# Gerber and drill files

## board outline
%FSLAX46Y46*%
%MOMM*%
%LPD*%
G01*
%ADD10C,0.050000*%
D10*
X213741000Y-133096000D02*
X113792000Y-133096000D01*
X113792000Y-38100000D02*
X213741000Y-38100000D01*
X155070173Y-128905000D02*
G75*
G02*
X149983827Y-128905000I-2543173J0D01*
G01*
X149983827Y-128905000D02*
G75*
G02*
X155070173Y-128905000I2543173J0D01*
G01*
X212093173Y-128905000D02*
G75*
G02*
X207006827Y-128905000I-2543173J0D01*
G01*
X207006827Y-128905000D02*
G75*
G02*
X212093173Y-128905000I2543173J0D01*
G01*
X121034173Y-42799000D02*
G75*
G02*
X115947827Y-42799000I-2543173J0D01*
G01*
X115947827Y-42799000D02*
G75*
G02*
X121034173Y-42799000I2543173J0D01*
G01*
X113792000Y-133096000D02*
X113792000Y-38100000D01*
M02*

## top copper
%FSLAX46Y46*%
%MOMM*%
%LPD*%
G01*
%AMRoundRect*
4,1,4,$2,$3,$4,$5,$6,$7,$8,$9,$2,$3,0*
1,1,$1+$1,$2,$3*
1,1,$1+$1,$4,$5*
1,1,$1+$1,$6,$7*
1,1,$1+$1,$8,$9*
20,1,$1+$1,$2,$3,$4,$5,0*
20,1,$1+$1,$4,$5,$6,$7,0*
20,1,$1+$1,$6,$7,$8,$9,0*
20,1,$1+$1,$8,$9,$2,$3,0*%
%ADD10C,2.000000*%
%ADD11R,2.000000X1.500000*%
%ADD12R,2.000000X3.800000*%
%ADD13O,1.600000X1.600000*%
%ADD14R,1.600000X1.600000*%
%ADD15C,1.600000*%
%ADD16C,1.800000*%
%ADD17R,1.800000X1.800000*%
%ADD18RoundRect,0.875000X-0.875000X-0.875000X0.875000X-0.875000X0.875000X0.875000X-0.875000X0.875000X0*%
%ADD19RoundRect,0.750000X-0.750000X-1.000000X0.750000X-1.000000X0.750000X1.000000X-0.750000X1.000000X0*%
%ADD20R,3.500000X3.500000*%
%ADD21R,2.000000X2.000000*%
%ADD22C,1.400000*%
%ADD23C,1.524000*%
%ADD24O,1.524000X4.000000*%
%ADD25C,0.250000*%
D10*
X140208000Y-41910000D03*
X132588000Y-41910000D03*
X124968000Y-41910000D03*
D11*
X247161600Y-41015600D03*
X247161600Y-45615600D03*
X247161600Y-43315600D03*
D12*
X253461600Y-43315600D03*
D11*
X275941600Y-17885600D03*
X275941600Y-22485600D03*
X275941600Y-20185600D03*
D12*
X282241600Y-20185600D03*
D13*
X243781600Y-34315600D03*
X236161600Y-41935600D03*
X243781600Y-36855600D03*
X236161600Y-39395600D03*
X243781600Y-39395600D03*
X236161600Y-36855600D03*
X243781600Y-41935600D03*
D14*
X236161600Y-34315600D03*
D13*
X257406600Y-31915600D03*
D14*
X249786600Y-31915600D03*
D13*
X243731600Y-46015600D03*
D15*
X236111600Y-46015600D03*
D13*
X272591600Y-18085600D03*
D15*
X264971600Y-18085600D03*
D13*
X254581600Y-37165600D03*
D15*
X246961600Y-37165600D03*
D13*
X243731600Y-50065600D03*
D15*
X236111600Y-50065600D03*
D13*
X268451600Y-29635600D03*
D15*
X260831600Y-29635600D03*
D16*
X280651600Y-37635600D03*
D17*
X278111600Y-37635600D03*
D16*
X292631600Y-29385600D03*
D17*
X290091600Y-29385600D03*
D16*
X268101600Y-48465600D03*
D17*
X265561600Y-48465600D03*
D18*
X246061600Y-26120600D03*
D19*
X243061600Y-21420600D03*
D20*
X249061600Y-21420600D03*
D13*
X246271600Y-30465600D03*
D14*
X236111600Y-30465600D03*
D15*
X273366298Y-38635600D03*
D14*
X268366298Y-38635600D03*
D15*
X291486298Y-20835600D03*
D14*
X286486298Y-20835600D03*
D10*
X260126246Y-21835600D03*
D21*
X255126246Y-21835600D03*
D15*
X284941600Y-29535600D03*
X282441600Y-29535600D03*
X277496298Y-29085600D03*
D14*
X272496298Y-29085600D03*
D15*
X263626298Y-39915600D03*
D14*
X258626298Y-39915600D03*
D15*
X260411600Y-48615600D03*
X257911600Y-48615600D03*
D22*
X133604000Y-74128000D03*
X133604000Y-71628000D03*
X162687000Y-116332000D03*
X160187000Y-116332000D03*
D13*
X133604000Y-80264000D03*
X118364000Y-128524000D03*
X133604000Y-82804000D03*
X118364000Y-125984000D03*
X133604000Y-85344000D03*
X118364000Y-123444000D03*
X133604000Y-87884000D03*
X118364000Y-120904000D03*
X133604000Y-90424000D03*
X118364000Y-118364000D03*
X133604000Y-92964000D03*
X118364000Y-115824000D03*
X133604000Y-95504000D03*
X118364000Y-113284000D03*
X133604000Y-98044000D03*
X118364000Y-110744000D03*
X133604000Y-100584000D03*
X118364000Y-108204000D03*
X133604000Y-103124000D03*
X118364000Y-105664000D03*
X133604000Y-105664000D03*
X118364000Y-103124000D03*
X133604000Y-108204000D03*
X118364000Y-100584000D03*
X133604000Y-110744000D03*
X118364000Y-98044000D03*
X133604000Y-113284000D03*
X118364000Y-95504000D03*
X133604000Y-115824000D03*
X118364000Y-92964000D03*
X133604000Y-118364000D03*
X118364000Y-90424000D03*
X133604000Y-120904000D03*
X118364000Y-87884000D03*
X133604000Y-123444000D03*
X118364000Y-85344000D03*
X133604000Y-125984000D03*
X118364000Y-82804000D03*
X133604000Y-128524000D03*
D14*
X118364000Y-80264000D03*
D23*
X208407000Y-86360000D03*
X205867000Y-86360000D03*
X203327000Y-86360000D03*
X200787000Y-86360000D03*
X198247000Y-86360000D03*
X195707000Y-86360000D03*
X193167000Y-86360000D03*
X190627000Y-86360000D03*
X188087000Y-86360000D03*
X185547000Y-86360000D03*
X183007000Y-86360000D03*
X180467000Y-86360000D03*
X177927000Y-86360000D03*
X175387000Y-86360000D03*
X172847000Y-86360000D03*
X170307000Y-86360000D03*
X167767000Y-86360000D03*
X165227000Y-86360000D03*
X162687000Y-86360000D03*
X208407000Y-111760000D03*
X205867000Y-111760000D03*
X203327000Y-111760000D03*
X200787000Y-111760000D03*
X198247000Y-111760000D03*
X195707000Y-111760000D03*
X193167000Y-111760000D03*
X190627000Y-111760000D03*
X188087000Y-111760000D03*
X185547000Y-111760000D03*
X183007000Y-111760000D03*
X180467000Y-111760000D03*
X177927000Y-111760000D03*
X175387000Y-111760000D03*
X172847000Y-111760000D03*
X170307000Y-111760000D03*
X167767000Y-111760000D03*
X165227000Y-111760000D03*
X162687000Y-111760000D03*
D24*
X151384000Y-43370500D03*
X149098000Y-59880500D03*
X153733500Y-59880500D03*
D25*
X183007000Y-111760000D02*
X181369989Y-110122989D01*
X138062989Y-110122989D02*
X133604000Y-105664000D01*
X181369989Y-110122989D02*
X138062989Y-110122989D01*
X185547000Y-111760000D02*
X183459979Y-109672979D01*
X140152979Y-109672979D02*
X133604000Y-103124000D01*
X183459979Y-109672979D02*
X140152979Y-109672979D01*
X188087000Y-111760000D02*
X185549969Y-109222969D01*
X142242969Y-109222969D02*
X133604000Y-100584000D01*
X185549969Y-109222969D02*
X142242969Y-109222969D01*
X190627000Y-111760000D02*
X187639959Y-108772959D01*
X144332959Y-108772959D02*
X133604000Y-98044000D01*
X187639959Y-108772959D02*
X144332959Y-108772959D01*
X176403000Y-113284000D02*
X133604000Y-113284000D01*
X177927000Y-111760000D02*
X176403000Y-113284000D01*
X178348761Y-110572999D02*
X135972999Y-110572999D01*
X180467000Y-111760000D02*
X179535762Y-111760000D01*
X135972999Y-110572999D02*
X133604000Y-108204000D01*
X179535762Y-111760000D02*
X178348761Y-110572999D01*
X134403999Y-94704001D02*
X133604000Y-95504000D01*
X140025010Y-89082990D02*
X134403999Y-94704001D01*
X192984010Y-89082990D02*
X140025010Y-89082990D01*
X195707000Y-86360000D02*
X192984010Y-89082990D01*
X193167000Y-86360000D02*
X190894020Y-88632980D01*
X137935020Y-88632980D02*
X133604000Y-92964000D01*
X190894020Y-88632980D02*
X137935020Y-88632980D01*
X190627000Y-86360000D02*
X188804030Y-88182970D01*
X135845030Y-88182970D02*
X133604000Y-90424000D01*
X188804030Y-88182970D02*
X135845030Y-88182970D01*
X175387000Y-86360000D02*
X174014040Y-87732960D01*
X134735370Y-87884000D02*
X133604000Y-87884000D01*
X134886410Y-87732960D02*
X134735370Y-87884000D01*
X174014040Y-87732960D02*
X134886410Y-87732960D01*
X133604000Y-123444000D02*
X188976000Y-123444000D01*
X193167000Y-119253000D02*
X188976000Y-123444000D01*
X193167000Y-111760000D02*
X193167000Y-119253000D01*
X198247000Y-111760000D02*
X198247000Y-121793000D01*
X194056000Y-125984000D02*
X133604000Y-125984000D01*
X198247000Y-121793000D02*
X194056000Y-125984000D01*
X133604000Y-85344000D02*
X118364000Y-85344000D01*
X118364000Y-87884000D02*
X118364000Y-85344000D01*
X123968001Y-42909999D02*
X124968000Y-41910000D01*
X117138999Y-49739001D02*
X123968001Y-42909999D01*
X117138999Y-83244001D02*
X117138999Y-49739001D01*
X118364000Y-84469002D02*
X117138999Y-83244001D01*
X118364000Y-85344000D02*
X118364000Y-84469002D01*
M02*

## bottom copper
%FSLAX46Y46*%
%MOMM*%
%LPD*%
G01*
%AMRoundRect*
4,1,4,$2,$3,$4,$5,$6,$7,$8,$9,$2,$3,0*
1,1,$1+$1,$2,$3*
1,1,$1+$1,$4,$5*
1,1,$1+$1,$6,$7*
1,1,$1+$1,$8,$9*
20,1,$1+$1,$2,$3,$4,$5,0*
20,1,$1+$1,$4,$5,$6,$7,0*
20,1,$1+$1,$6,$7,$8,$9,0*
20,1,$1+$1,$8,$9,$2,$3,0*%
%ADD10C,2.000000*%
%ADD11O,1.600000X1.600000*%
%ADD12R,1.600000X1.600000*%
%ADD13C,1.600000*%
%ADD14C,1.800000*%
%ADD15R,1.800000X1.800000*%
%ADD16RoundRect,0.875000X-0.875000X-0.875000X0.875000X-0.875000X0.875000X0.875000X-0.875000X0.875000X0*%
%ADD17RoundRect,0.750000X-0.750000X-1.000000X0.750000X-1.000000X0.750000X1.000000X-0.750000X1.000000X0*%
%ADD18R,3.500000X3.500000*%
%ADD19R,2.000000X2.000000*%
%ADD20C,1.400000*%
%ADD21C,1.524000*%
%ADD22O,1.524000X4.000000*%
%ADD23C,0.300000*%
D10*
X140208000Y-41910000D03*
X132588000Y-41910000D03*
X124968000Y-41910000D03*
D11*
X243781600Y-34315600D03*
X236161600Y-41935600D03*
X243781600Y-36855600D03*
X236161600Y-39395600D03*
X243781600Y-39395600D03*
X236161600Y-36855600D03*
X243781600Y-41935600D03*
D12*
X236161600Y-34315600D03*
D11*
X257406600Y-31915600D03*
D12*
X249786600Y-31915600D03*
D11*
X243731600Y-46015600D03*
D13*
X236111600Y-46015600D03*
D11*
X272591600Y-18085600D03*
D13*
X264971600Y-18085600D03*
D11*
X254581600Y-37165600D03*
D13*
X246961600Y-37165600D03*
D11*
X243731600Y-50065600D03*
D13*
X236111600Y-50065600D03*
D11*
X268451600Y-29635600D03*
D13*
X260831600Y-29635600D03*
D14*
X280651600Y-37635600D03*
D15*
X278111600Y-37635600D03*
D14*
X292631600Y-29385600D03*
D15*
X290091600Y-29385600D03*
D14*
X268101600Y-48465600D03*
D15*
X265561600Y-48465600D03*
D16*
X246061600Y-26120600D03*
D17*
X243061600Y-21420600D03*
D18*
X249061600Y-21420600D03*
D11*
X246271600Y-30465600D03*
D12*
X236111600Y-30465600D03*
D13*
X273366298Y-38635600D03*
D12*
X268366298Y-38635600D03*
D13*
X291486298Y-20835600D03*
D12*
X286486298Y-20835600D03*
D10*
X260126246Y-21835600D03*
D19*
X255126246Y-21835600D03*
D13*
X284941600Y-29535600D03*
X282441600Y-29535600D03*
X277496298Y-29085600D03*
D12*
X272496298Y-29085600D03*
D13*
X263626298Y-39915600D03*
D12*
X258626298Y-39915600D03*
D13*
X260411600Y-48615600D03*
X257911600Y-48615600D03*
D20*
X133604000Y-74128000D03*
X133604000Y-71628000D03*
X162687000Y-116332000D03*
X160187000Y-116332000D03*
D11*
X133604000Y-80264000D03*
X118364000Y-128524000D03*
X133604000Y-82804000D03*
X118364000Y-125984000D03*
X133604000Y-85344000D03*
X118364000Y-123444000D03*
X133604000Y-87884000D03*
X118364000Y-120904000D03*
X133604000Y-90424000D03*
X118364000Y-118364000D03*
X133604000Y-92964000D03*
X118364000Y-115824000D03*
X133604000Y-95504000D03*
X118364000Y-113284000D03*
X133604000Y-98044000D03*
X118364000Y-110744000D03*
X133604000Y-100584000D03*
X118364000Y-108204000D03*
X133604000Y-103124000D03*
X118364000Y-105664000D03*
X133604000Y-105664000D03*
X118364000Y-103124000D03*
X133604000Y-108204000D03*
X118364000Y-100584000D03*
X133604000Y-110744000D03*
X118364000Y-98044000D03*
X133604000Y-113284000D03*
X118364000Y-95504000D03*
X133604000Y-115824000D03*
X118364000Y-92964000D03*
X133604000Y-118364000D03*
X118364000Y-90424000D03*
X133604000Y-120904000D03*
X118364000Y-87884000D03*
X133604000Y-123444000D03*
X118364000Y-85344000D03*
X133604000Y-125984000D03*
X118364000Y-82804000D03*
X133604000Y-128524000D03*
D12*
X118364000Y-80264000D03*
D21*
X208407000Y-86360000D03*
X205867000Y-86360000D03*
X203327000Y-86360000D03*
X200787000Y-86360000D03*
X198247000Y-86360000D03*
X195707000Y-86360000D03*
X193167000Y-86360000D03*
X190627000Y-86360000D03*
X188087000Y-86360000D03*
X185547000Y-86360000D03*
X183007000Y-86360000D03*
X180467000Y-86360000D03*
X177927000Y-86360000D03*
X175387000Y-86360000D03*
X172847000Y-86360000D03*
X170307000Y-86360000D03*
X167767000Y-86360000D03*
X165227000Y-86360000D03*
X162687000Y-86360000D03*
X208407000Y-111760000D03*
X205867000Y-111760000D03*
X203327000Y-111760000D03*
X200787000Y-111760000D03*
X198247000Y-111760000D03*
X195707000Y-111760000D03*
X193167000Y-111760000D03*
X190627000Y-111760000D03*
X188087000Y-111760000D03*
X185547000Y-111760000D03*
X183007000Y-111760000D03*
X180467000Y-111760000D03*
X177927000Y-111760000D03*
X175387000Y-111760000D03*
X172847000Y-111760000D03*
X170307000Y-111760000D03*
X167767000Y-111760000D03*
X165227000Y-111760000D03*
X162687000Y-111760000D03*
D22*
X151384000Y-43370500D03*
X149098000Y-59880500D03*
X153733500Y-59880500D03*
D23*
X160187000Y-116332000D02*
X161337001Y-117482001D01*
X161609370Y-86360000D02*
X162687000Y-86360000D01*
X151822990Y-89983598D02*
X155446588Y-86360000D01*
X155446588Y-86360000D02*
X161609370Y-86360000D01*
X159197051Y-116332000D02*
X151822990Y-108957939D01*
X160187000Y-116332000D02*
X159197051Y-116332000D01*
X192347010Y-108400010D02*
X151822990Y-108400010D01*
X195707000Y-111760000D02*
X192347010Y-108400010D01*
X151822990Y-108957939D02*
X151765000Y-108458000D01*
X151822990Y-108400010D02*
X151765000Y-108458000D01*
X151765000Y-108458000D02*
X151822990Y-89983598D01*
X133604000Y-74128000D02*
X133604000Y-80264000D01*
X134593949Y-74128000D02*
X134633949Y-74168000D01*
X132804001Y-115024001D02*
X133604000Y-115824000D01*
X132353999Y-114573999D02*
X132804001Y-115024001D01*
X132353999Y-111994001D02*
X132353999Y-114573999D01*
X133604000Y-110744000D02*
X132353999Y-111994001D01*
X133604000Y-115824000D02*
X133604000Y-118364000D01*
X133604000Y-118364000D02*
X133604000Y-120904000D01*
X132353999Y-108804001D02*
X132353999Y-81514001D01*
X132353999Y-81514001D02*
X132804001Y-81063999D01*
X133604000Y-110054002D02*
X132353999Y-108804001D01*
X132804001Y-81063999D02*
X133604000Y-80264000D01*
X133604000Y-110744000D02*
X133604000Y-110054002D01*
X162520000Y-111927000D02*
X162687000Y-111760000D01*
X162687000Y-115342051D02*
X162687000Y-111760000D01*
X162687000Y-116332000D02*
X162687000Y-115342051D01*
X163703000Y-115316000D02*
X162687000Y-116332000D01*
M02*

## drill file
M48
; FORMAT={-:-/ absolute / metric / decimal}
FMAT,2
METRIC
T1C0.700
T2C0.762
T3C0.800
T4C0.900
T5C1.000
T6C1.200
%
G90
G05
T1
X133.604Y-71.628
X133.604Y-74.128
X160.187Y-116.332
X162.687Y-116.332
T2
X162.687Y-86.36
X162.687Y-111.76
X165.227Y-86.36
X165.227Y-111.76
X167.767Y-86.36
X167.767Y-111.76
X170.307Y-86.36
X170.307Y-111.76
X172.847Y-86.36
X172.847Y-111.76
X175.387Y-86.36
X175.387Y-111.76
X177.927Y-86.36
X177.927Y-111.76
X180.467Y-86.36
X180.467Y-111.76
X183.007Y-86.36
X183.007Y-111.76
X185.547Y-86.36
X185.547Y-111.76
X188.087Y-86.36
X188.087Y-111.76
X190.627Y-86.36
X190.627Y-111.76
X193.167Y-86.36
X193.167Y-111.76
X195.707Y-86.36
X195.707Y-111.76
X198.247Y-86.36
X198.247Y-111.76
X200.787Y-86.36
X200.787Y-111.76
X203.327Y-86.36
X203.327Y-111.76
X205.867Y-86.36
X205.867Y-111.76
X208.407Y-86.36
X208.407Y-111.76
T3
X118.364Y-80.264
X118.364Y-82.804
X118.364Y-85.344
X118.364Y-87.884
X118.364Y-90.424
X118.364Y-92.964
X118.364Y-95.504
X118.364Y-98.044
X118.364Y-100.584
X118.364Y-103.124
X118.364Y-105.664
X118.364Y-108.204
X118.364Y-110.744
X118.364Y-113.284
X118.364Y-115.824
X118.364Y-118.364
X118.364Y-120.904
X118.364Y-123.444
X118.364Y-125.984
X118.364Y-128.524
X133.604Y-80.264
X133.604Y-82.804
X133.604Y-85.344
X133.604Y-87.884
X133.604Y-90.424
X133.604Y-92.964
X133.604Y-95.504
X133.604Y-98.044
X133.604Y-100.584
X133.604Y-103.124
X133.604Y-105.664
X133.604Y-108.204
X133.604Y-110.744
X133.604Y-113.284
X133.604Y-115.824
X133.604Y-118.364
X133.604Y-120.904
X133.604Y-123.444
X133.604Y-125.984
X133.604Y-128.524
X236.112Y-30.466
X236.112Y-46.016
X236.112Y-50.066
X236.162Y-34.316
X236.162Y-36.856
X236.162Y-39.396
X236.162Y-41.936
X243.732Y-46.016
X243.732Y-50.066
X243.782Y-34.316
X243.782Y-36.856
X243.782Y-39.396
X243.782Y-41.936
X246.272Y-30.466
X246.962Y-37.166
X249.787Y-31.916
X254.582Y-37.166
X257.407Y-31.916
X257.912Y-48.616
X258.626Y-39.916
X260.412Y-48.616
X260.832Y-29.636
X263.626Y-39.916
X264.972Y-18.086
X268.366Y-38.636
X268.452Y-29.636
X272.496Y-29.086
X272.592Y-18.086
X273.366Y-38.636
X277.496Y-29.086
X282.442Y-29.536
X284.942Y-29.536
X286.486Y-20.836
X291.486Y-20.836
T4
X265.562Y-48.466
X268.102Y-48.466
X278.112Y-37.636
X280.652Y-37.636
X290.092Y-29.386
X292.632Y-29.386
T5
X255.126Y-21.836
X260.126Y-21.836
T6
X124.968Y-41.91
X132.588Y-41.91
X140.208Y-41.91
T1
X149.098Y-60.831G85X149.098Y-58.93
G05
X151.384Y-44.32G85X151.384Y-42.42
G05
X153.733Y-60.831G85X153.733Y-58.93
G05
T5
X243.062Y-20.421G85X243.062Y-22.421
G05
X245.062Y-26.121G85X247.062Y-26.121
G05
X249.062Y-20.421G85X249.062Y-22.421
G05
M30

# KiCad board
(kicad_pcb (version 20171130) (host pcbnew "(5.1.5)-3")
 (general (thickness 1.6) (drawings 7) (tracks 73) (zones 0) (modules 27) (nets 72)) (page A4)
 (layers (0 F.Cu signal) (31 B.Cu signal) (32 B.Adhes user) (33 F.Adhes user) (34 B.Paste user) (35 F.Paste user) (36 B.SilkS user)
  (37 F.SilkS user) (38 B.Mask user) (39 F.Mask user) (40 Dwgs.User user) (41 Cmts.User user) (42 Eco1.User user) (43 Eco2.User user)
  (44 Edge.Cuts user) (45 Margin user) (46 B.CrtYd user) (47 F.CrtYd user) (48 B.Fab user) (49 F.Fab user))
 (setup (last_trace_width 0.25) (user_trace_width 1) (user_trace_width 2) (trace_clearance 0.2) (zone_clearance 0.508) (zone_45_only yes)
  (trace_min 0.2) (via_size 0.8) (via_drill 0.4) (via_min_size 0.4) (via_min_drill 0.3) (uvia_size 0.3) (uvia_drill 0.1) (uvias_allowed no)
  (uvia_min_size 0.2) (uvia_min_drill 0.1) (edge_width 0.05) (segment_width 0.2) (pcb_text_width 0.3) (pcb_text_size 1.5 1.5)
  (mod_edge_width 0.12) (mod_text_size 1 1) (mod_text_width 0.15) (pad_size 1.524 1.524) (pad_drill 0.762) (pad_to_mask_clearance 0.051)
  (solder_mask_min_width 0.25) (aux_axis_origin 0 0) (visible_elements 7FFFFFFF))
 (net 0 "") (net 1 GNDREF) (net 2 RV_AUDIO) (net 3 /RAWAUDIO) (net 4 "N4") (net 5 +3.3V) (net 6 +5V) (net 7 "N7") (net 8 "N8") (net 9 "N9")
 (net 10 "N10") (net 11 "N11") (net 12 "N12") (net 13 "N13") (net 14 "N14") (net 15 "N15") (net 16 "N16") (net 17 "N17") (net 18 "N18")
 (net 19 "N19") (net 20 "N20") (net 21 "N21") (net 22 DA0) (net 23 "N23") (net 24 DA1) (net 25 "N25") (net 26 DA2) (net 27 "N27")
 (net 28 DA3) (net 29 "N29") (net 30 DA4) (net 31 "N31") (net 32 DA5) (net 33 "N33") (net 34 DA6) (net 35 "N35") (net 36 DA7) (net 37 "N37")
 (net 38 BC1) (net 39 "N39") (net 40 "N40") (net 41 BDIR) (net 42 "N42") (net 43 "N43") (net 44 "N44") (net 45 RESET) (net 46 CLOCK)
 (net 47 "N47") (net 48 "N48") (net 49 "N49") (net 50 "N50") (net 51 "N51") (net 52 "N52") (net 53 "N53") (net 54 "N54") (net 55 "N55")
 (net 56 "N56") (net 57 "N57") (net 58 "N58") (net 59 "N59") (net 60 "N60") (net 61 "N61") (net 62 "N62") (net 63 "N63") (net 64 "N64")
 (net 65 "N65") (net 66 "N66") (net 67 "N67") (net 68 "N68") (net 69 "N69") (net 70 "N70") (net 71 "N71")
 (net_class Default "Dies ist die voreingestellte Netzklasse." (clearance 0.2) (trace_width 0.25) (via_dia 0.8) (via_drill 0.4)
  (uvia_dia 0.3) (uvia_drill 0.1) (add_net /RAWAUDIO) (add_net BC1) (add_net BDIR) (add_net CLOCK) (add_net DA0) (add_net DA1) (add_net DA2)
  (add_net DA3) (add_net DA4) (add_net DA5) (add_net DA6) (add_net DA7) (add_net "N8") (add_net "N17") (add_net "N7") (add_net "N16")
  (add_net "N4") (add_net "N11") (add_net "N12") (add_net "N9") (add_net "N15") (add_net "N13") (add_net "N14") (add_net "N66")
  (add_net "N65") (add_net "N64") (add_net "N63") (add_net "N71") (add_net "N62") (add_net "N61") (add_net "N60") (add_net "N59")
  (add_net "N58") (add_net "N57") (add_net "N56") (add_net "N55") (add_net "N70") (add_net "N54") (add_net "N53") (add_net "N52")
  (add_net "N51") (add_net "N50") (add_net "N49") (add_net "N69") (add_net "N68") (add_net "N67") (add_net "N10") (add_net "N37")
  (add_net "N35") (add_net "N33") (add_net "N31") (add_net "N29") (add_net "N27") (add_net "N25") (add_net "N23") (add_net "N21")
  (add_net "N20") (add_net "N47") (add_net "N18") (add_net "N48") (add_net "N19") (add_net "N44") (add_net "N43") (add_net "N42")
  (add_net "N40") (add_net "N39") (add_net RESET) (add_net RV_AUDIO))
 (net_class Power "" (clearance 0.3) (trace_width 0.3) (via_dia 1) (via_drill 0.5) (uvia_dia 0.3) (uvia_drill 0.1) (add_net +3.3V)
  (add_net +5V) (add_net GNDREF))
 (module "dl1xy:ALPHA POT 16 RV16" (layer F.Cu) (at 132.588 46.863 180)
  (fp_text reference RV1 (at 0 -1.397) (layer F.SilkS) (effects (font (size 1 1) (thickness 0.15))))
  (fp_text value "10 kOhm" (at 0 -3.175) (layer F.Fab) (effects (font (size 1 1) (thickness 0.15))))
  (pad 1 thru_hole circle (at -7.62 4.953 180) (size 2 2) (drill 1.2) (layers *.Cu *.Mask) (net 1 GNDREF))
  (pad 2 thru_hole circle (at 0 4.953 180) (size 2 2) (drill 1.2) (layers *.Cu *.Mask) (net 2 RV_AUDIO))
  (pad 3 thru_hole circle (at 7.62 4.953 180) (size 2 2) (drill 1.2) (layers *.Cu *.Mask) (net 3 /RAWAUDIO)))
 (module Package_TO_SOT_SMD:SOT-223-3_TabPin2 (layer F.Cu) (at 250.3116 43.3156)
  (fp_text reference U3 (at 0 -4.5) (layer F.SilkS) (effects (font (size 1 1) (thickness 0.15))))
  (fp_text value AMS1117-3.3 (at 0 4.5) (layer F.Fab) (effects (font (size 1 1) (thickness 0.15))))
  (pad 1 smd rect (at -3.15 -2.3) (size 2 1.5) (layers F.Cu F.Paste F.Mask) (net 1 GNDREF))
  (pad 3 smd rect (at -3.15 2.3) (size 2 1.5) (layers F.Cu F.Paste F.Mask) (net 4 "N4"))
  (pad 2 smd rect (at -3.15 0) (size 2 1.5) (layers F.Cu F.Paste F.Mask) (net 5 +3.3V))
  (pad 2 smd rect (at 3.15 0) (size 2 3.8) (layers F.Cu F.Paste F.Mask) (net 5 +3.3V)))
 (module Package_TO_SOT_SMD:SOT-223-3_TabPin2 (layer F.Cu) (at 279.0916 20.1856)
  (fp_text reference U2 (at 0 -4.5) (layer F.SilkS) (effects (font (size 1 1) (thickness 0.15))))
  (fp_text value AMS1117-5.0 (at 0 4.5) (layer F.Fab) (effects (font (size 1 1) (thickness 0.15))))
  (pad 1 smd rect (at -3.15 -2.3) (size 2 1.5) (layers F.Cu F.Paste F.Mask) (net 1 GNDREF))
  (pad 3 smd rect (at -3.15 2.3) (size 2 1.5) (layers F.Cu F.Paste F.Mask) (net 4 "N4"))
  (pad 2 smd rect (at -3.15 0) (size 2 1.5) (layers F.Cu F.Paste F.Mask) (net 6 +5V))
  (pad 2 smd rect (at 3.15 0) (size 2 3.8) (layers F.Cu F.Paste F.Mask) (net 6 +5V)))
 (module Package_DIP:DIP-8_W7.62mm (layer F.Cu) (at 236.1616 34.3156)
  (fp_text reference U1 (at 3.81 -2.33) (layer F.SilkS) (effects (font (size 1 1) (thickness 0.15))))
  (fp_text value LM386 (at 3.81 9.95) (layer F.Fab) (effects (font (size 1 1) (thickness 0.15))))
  (pad 8 thru_hole oval (at 7.62 0) (size 1.6 1.6) (drill 0.8) (layers *.Cu *.Mask) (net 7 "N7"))
  (pad 4 thru_hole oval (at 0 7.62) (size 1.6 1.6) (drill 0.8) (layers *.Cu *.Mask) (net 1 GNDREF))
  (pad 7 thru_hole oval (at 7.62 2.54) (size 1.6 1.6) (drill 0.8) (layers *.Cu *.Mask) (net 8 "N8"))
  (pad 3 thru_hole oval (at 0 5.08) (size 1.6 1.6) (drill 0.8) (layers *.Cu *.Mask) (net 2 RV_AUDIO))
  (pad 6 thru_hole oval (at 7.62 5.08) (size 1.6 1.6) (drill 0.8) (layers *.Cu *.Mask) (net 6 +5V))
  (pad 2 thru_hole oval (at 0 2.54) (size 1.6 1.6) (drill 0.8) (layers *.Cu *.Mask) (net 1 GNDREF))
  (pad 5 thru_hole oval (at 7.62 7.62) (size 1.6 1.6) (drill 0.8) (layers *.Cu *.Mask) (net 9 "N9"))
  (pad 1 thru_hole rect (at 0 0) (size 1.6 1.6) (drill 0.8) (layers *.Cu *.Mask) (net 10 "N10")))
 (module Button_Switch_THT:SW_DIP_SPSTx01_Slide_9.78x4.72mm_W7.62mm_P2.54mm (layer F.Cu) (at 249.7866 31.9156)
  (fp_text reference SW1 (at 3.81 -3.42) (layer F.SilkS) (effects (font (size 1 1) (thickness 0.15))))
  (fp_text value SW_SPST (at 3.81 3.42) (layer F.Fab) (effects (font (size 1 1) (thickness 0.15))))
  (pad 2 thru_hole oval (at 7.62 0) (size 1.6 1.6) (drill 0.8) (layers *.Cu *.Mask) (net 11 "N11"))
  (pad 1 thru_hole rect (at 0 0) (size 1.6 1.6) (drill 0.8) (layers *.Cu *.Mask) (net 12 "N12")))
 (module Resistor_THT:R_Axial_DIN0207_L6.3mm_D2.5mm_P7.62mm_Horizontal (layer F.Cu) (at 236.1116 46.0156)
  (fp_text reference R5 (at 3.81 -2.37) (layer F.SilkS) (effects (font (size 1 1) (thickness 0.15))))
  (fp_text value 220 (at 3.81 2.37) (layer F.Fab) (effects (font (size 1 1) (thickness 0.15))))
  (pad 2 thru_hole oval (at 7.62 0) (size 1.6 1.6) (drill 0.8) (layers *.Cu *.Mask) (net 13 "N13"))
  (pad 1 thru_hole circle (at 0 0) (size 1.6 1.6) (drill 0.8) (layers *.Cu *.Mask) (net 5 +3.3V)))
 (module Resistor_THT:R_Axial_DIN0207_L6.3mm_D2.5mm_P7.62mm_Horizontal (layer F.Cu) (at 264.9716 18.0856)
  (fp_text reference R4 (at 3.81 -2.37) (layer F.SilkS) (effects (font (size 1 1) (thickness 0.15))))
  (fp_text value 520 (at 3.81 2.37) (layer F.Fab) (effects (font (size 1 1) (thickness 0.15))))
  (pad 2 thru_hole oval (at 7.62 0) (size 1.6 1.6) (drill 0.8) (layers *.Cu *.Mask) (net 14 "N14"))
  (pad 1 thru_hole circle (at 0 0) (size 1.6 1.6) (drill 0.8) (layers *.Cu *.Mask) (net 6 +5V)))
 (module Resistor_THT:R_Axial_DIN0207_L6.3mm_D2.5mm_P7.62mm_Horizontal (layer F.Cu) (at 246.9616 37.1656)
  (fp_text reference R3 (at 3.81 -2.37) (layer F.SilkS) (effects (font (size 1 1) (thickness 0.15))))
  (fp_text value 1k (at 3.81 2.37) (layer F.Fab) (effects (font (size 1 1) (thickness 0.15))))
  (pad 2 thru_hole oval (at 7.62 0) (size 1.6 1.6) (drill 0.8) (layers *.Cu *.Mask) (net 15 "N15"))
  (pad 1 thru_hole circle (at 0 0) (size 1.6 1.6) (drill 0.8) (layers *.Cu *.Mask) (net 11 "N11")))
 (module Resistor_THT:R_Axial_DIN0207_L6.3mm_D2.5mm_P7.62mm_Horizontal (layer F.Cu) (at 236.1116 50.0656)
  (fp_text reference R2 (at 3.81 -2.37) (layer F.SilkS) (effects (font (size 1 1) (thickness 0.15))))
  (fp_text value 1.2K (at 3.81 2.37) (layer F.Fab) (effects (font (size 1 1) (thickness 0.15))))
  (pad 2 thru_hole oval (at 7.62 0) (size 1.6 1.6) (drill 0.8) (layers *.Cu *.Mask) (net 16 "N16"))
  (pad 1 thru_hole circle (at 0 0) (size 1.6 1.6) (drill 0.8) (layers *.Cu *.Mask) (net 9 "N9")))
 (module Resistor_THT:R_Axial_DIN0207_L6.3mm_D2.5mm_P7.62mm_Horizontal (layer F.Cu) (at 260.8316 29.6356)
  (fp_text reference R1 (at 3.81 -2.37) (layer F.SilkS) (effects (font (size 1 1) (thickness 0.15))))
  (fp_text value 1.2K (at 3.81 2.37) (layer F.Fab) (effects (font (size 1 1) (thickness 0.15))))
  (pad 2 thru_hole oval (at 7.62 0) (size 1.6 1.6) (drill 0.8) (layers *.Cu *.Mask) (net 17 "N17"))
  (pad 1 thru_hole circle (at 0 0) (size 1.6 1.6) (drill 0.8) (layers *.Cu *.Mask) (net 10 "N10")))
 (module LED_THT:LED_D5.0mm (layer F.Cu) (at 278.1116 37.6356)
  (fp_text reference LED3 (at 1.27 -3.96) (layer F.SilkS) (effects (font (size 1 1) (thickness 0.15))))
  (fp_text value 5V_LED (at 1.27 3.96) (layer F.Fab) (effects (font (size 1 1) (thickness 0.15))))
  (pad 2 thru_hole circle (at 2.54 0) (size 1.8 1.8) (drill 0.9) (layers *.Cu *.Mask) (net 14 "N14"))
  (pad 1 thru_hole rect (at 0 0) (size 1.8 1.8) (drill 0.9) (layers *.Cu *.Mask) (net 1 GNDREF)))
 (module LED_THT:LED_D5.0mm (layer F.Cu) (at 290.0916 29.3856)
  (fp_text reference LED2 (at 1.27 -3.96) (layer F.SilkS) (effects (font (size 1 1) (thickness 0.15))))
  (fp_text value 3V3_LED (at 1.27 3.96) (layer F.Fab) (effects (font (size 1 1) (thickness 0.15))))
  (pad 2 thru_hole circle (at 2.54 0) (size 1.8 1.8) (drill 0.9) (layers *.Cu *.Mask) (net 13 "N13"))
  (pad 1 thru_hole rect (at 0 0) (size 1.8 1.8) (drill 0.9) (layers *.Cu *.Mask) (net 1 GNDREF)))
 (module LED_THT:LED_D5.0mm (layer F.Cu) (at 265.5616 48.4656)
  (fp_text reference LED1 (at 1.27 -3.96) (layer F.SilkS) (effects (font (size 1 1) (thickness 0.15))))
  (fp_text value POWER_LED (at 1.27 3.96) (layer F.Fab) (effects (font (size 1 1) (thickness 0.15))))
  (pad 2 thru_hole circle (at 2.54 0) (size 1.8 1.8) (drill 0.9) (layers *.Cu *.Mask) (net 15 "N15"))
  (pad 1 thru_hole rect (at 0 0) (size 1.8 1.8) (drill 0.9) (layers *.Cu *.Mask) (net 1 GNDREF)))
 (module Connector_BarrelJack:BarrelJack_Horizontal (layer F.Cu) (at 249.0616 21.4206)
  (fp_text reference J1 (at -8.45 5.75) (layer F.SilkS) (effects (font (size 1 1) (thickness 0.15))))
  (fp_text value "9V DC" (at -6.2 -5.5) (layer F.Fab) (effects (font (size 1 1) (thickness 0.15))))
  (pad 3 thru_hole roundrect (at -3 4.7) (size 3.5 3.5) (drill oval 3 1) (layers *.Cu *.Mask) (roundrect_rratio 0.25))
  (pad 2 thru_hole roundrect (at -6 0) (size 3 3.5) (drill oval 1 3) (layers *.Cu *.Mask) (roundrect_rratio 0.25) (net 1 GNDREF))
  (pad 1 thru_hole rect (at 0 0) (size 3.5 3.5) (drill oval 1 3) (layers *.Cu *.Mask) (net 12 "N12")))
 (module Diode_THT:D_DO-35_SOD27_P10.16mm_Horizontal (layer F.Cu) (at 236.1116 30.4656)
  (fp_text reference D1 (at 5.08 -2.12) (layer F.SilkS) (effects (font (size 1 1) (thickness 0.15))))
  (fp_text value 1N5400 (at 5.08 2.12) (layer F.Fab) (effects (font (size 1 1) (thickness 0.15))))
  (pad 2 thru_hole oval (at 10.16 0) (size 1.6 1.6) (drill 0.8) (layers *.Cu *.Mask) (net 11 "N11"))
  (pad 1 thru_hole rect (at 0 0) (size 1.6 1.6) (drill 0.8) (layers *.Cu *.Mask) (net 4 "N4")))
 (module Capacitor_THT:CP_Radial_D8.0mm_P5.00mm (layer F.Cu) (at 268.366298 38.6356)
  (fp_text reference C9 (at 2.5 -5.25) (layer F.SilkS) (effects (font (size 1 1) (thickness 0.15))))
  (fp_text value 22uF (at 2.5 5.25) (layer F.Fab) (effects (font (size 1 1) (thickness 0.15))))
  (pad 2 thru_hole circle (at 5 0) (size 1.6 1.6) (drill 0.8) (layers *.Cu *.Mask) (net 1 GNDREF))
  (pad 1 thru_hole rect (at 0 0) (size 1.6 1.6) (drill 0.8) (layers *.Cu *.Mask) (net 5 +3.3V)))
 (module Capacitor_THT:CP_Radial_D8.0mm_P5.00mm (layer F.Cu) (at 286.486298 20.8356)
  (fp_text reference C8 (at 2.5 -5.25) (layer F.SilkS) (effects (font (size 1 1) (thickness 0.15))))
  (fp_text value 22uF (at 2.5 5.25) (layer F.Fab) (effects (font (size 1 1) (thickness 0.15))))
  (pad 2 thru_hole circle (at 5 0) (size 1.6 1.6) (drill 0.8) (layers *.Cu *.Mask) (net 1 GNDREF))
  (pad 1 thru_hole rect (at 0 0) (size 1.6 1.6) (drill 0.8) (layers *.Cu *.Mask) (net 6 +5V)))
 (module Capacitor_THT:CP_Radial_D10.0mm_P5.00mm (layer F.Cu) (at 255.126246 21.8356)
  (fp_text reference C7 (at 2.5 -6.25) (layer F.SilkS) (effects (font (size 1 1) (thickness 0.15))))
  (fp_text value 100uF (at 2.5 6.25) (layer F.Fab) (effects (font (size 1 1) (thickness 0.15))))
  (pad 2 thru_hole circle (at 5 0) (size 2 2) (drill 1) (layers *.Cu *.Mask) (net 1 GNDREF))
  (pad 1 thru_hole rect (at 0 0) (size 2 2) (drill 1) (layers *.Cu *.Mask) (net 4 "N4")))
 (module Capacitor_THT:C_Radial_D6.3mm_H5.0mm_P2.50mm (layer F.Cu) (at 282.4416 29.5356)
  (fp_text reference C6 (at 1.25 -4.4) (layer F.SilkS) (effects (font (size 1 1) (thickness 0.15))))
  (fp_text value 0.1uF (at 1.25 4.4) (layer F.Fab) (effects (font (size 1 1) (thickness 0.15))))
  (pad 2 thru_hole circle (at 2.5 0) (size 1.6 1.6) (drill 0.8) (layers *.Cu *.Mask) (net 1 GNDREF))
  (pad 1 thru_hole circle (at 0 0) (size 1.6 1.6) (drill 0.8) (layers *.Cu *.Mask) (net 16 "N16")))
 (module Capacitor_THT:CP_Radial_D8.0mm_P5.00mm (layer F.Cu) (at 272.496298 29.0856)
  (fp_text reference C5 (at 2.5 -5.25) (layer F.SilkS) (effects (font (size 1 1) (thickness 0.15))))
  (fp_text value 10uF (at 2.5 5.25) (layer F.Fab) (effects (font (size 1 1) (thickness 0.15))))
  (pad 2 thru_hole circle (at 5 0) (size 1.6 1.6) (drill 0.8) (layers *.Cu *.Mask) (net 7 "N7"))
  (pad 1 thru_hole rect (at 0 0) (size 1.6 1.6) (drill 0.8) (layers *.Cu *.Mask) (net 17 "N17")))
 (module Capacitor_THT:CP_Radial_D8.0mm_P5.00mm (layer F.Cu) (at 258.626298 39.9156)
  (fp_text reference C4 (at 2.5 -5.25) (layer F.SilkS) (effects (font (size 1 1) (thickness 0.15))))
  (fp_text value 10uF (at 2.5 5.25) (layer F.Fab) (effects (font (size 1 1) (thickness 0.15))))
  (pad 2 thru_hole circle (at 5 0) (size 1.6 1.6) (drill 0.8) (layers *.Cu *.Mask) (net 1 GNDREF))
  (pad 1 thru_hole rect (at 0 0) (size 1.6 1.6) (drill 0.8) (layers *.Cu *.Mask) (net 8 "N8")))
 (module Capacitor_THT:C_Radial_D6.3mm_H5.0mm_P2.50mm (layer F.Cu) (at 257.9116 48.6156)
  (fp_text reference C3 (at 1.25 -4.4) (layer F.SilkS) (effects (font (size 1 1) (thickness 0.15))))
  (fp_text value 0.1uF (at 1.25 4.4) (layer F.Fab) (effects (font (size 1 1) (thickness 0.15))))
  (pad 2 thru_hole circle (at 2.5 0) (size 1.6 1.6) (drill 0.8) (layers *.Cu *.Mask) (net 6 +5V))
  (pad 1 thru_hole circle (at 0 0) (size 1.6 1.6) (drill 0.8) (layers *.Cu *.Mask) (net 1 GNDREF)))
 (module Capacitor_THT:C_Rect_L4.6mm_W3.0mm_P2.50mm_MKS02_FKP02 (layer F.Cu) (at 133.604 71.628 270)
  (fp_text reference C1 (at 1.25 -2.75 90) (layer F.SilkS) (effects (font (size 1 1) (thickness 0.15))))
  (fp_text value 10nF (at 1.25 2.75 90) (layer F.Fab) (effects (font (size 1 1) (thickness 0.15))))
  (pad 2 thru_hole circle (at 2.5 0 270) (size 1.4 1.4) (drill 0.7) (layers *.Cu *.Mask) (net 6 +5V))
  (pad 1 thru_hole circle (at 0 0 270) (size 1.4 1.4) (drill 0.7) (layers *.Cu *.Mask) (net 1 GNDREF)))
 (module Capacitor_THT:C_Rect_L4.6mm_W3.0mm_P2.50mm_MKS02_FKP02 (layer F.Cu) (at 160.187 116.332)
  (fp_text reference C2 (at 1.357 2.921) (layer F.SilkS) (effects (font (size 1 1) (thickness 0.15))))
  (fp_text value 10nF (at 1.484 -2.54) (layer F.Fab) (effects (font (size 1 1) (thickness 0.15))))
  (pad 2 thru_hole circle (at 2.5 0) (size 1.4 1.4) (drill 0.7) (layers *.Cu *.Mask) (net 5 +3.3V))
  (pad 1 thru_hole circle (at 0 0) (size 1.4 1.4) (drill 0.7) (layers *.Cu *.Mask) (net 1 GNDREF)))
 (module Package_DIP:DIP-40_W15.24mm (layer F.Cu) (at 118.364 80.264)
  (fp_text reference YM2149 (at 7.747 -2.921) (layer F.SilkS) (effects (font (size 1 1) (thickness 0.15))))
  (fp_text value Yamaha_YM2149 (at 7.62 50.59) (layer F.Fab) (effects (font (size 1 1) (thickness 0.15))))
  (pad 40 thru_hole oval (at 15.24 0) (size 1.6 1.6) (drill 0.8) (layers *.Cu *.Mask) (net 6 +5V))
  (pad 20 thru_hole oval (at 0 48.26) (size 1.6 1.6) (drill 0.8) (layers *.Cu *.Mask) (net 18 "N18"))
  (pad 39 thru_hole oval (at 15.24 2.54) (size 1.6 1.6) (drill 0.8) (layers *.Cu *.Mask) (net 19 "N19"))
  (pad 19 thru_hole oval (at 0 45.72) (size 1.6 1.6) (drill 0.8) (layers *.Cu *.Mask) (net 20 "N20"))
  (pad 38 thru_hole oval (at 15.24 5.08) (size 1.6 1.6) (drill 0.8) (layers *.Cu *.Mask) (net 3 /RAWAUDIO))
  (pad 18 thru_hole oval (at 0 43.18) (size 1.6 1.6) (drill 0.8) (layers *.Cu *.Mask) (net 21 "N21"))
  (pad 37 thru_hole oval (at 15.24 7.62) (size 1.6 1.6) (drill 0.8) (layers *.Cu *.Mask) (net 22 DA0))
  (pad 17 thru_hole oval (at 0 40.64) (size 1.6 1.6) (drill 0.8) (layers *.Cu *.Mask) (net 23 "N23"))
  (pad 36 thru_hole oval (at 15.24 10.16) (size 1.6 1.6) (drill 0.8) (layers *.Cu *.Mask) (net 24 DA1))
  (pad 16 thru_hole oval (at 0 38.1) (size 1.6 1.6) (drill 0.8) (layers *.Cu *.Mask) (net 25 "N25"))
  (pad 35 thru_hole oval (at 15.24 12.7) (size 1.6 1.6) (drill 0.8) (layers *.Cu *.Mask) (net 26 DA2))
  (pad 15 thru_hole oval (at 0 35.56) (size 1.6 1.6) (drill 0.8) (layers *.Cu *.Mask) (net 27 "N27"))
  (pad 34 thru_hole oval (at 15.24 15.24) (size 1.6 1.6) (drill 0.8) (layers *.Cu *.Mask) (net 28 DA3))
  (pad 14 thru_hole oval (at 0 33.02) (size 1.6 1.6) (drill 0.8) (layers *.Cu *.Mask) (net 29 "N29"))
  (pad 33 thru_hole oval (at 15.24 17.78) (size 1.6 1.6) (drill 0.8) (layers *.Cu *.Mask) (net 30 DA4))
  (pad 13 thru_hole oval (at 0 30.48) (size 1.6 1.6) (drill 0.8) (layers *.Cu *.Mask) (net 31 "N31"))
  (pad 32 thru_hole oval (at 15.24 20.32) (size 1.6 1.6) (drill 0.8) (layers *.Cu *.Mask) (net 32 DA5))
  (pad 12 thru_hole oval (at 0 27.94) (size 1.6 1.6) (drill 0.8) (layers *.Cu *.Mask) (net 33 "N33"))
  (pad 31 thru_hole oval (at 15.24 22.86) (size 1.6 1.6) (drill 0.8) (layers *.Cu *.Mask) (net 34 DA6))
  (pad 11 thru_hole oval (at 0 25.4) (size 1.6 1.6) (drill 0.8) (layers *.Cu *.Mask) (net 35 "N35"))
  (pad 30 thru_hole oval (at 15.24 25.4) (size 1.6 1.6) (drill 0.8) (layers *.Cu *.Mask) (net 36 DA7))
  (pad 10 thru_hole oval (at 0 22.86) (size 1.6 1.6) (drill 0.8) (layers *.Cu *.Mask) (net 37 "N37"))
  (pad 29 thru_hole oval (at 15.24 27.94) (size 1.6 1.6) (drill 0.8) (layers *.Cu *.Mask) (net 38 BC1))
  (pad 9 thru_hole oval (at 0 20.32) (size 1.6 1.6) (drill 0.8) (layers *.Cu *.Mask) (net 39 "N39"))
  (pad 28 thru_hole oval (at 15.24 30.48) (size 1.6 1.6) (drill 0.8) (layers *.Cu *.Mask) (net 6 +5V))
  (pad 8 thru_hole oval (at 0 17.78) (size 1.6 1.6) (drill 0.8) (layers *.Cu *.Mask) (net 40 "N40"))
  (pad 27 thru_hole oval (at 15.24 33.02) (size 1.6 1.6) (drill 0.8) (layers *.Cu *.Mask) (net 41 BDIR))
  (pad 7 thru_hole oval (at 0 15.24) (size 1.6 1.6) (drill 0.8) (layers *.Cu *.Mask) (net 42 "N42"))
  (pad 26 thru_hole oval (at 15.24 35.56) (size 1.6 1.6) (drill 0.8) (layers *.Cu *.Mask) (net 6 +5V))
  (pad 6 thru_hole oval (at 0 12.7) (size 1.6 1.6) (drill 0.8) (layers *.Cu *.Mask) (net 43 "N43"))
  (pad 25 thru_hole oval (at 15.24 38.1) (size 1.6 1.6) (drill 0.8) (layers *.Cu *.Mask) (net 6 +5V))
  (pad 5 thru_hole oval (at 0 10.16) (size 1.6 1.6) (drill 0.8) (layers *.Cu *.Mask) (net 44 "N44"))
  (pad 24 thru_hole oval (at 15.24 40.64) (size 1.6 1.6) (drill 0.8) (layers *.Cu *.Mask) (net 6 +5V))
  (pad 4 thru_hole oval (at 0 7.62) (size 1.6 1.6) (drill 0.8) (layers *.Cu *.Mask) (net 3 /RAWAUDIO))
  (pad 23 thru_hole oval (at 15.24 43.18) (size 1.6 1.6) (drill 0.8) (layers *.Cu *.Mask) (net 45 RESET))
  (pad 3 thru_hole oval (at 0 5.08) (size 1.6 1.6) (drill 0.8) (layers *.Cu *.Mask) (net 3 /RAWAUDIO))
  (pad 22 thru_hole oval (at 15.24 45.72) (size 1.6 1.6) (drill 0.8) (layers *.Cu *.Mask) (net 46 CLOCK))
  (pad 2 thru_hole oval (at 0 2.54) (size 1.6 1.6) (drill 0.8) (layers *.Cu *.Mask) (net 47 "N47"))
  (pad 21 thru_hole oval (at 15.24 48.26) (size 1.6 1.6) (drill 0.8) (layers *.Cu *.Mask) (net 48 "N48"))
  (pad 1 thru_hole rect (at 0 0) (size 1.6 1.6) (drill 0.8) (layers *.Cu *.Mask) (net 1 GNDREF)))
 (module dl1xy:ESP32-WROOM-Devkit (layer F.Cu) (at 154.432 99.06 90)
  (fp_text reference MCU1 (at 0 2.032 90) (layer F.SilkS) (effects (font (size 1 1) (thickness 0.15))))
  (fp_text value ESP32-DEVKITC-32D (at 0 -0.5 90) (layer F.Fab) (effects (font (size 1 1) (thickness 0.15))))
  (pad 38 thru_hole circle (at 12.7 53.975 270) (size 1.524 1.524) (drill 0.762) (layers *.Cu *.Mask) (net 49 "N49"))
  (pad 37 thru_hole circle (at 12.7 51.435 270) (size 1.524 1.524) (drill 0.762) (layers *.Cu *.Mask) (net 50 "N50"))
  (pad 36 thru_hole circle (at 12.7 48.895 270) (size 1.524 1.524) (drill 0.762) (layers *.Cu *.Mask) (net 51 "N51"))
  (pad 35 thru_hole circle (at 12.7 46.355 270) (size 1.524 1.524) (drill 0.762) (layers *.Cu *.Mask) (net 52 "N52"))
  (pad 34 thru_hole circle (at 12.7 43.815 270) (size 1.524 1.524) (drill 0.762) (layers *.Cu *.Mask) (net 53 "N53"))
  (pad 33 thru_hole circle (at 12.7 41.275 270) (size 1.524 1.524) (drill 0.762) (layers *.Cu *.Mask) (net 28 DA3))
  (pad 32 thru_hole circle (at 12.7 38.735 270) (size 1.524 1.524) (drill 0.762) (layers *.Cu *.Mask) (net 26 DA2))
  (pad 31 thru_hole circle (at 12.7 36.195 270) (size 1.524 1.524) (drill 0.762) (layers *.Cu *.Mask) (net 24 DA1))
  (pad 30 thru_hole circle (at 12.7 33.655 270) (size 1.524 1.524) (drill 0.762) (layers *.Cu *.Mask) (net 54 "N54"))
  (pad 29 thru_hole circle (at 12.7 31.115 270) (size 1.524 1.524) (drill 0.762) (layers *.Cu *.Mask) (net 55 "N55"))
  (pad 28 thru_hole circle (at 12.7 28.575 270) (size 1.524 1.524) (drill 0.762) (layers *.Cu *.Mask) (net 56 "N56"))
  (pad 27 thru_hole circle (at 12.7 26.035 270) (size 1.524 1.524) (drill 0.762) (layers *.Cu *.Mask) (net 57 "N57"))
  (pad 26 thru_hole circle (at 12.7 23.495 270) (size 1.524 1.524) (drill 0.762) (layers *.Cu *.Mask) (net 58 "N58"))
  (pad 25 thru_hole circle (at 12.7 20.955 270) (size 1.524 1.524) (drill 0.762) (layers *.Cu *.Mask) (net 22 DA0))
  (pad 24 thru_hole circle (at 12.7 18.415 270) (size 1.524 1.524) (drill 0.762) (layers *.Cu *.Mask) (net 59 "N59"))
  (pad 23 thru_hole circle (at 12.7 15.875 270) (size 1.524 1.524) (drill 0.762) (layers *.Cu *.Mask) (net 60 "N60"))
  (pad 22 thru_hole circle (at 12.7 13.335 270) (size 1.524 1.524) (drill 0.762) (layers *.Cu *.Mask) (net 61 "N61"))
  (pad 21 thru_hole circle (at 12.7 10.795 270) (size 1.524 1.524) (drill 0.762) (layers *.Cu *.Mask) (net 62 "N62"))
  (pad 20 thru_hole circle (at 12.7 8.255 270) (size 1.524 1.524) (drill 0.762) (layers *.Cu *.Mask) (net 1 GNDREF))
  (pad 19 thru_hole circle (at -12.7 53.975 90) (size 1.524 1.524) (drill 0.762) (layers *.Cu *.Mask) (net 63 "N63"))
  (pad 18 thru_hole circle (at -12.7 51.435 90) (size 1.524 1.524) (drill 0.762) (layers *.Cu *.Mask) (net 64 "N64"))
  (pad 17 thru_hole circle (at -12.7 48.895 90) (size 1.524 1.524) (drill 0.762) (layers *.Cu *.Mask) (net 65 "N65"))
  (pad 16 thru_hole circle (at -12.7 46.355 90) (size 1.524 1.524) (drill 0.762) (layers *.Cu *.Mask) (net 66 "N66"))
  (pad 15 thru_hole circle (at -12.7 43.815 90) (size 1.524 1.524) (drill 0.762) (layers *.Cu *.Mask) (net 46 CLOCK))
  (pad 14 thru_hole circle (at -12.7 41.275 90) (size 1.524 1.524) (drill 0.762) (layers *.Cu *.Mask) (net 1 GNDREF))
  (pad 13 thru_hole circle (at -12.7 38.735 90) (size 1.524 1.524) (drill 0.762) (layers *.Cu *.Mask) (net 45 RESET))
  (pad 12 thru_hole circle (at -12.7 36.195 90) (size 1.524 1.524) (drill 0.762) (layers *.Cu *.Mask) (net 30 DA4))
  (pad 11 thru_hole circle (at -12.7 33.655 90) (size 1.524 1.524) (drill 0.762) (layers *.Cu *.Mask) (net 32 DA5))
  (pad 10 thru_hole circle (at -12.7 31.115 90) (size 1.524 1.524) (drill 0.762) (layers *.Cu *.Mask) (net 34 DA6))
  (pad 9 thru_hole circle (at -12.7 28.575 90) (size 1.524 1.524) (drill 0.762) (layers *.Cu *.Mask) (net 36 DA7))
  (pad 8 thru_hole circle (at -12.7 26.035 90) (size 1.524 1.524) (drill 0.762) (layers *.Cu *.Mask) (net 38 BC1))
  (pad 7 thru_hole circle (at -12.7 23.495 90) (size 1.524 1.524) (drill 0.762) (layers *.Cu *.Mask) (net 41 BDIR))
  (pad 6 thru_hole circle (at -12.7 20.955 90) (size 1.524 1.524) (drill 0.762) (layers *.Cu *.Mask) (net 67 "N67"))
  (pad 5 thru_hole circle (at -12.7 18.415 90) (size 1.524 1.524) (drill 0.762) (layers *.Cu *.Mask) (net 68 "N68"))
  (pad 4 thru_hole circle (at -12.7 15.875 90) (size 1.524 1.524) (drill 0.762) (layers *.Cu *.Mask) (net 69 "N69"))
  (pad 3 thru_hole circle (at -12.7 13.335 90) (size 1.524 1.524) (drill 0.762) (layers *.Cu *.Mask) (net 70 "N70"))
  (pad 2 thru_hole circle (at -12.7 10.795 90) (size 1.524 1.524) (drill 0.762) (layers *.Cu *.Mask) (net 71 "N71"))
  (pad 1 thru_hole circle (at -12.7 8.255 90) (size 1.524 1.524) (drill 0.762) (layers *.Cu *.Mask) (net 5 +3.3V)))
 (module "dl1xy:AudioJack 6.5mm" (layer F.Cu) (at 151.384 66.548 180)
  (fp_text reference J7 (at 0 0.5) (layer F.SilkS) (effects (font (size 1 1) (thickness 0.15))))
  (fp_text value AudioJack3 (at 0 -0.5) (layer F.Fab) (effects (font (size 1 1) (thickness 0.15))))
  (pad S thru_hole oval (at 0 23.1775 180) (size 1.524 4) (drill oval 0.7 2.6) (layers *.Cu *.Mask) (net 1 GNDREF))
  (pad T thru_hole oval (at 2.286 6.6675 180) (size 1.524 4) (drill oval 0.7 2.6) (layers *.Cu *.Mask) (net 9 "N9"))
  (pad R thru_hole oval (at -2.3495 6.6675 180) (size 1.524 4) (drill oval 0.7 2.6) (layers *.Cu *.Mask) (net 9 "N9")))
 (gr_line (start 213.741 133.096) (end 113.792 133.096) (layer Edge.Cuts) (width 0.05))
 (gr_line (start 113.792 38.1) (end 213.741 38.1) (layer Edge.Cuts) (width 0.05))
 (gr_circle (center 152.527 128.905) (end 155.067 128.778) (layer Edge.Cuts) (width 0.05))
 (gr_circle (center 209.55 128.905) (end 212.09 128.778) (layer Edge.Cuts) (width 0.05))
 (gr_circle (center 118.491 42.799) (end 121.031 42.672) (layer Edge.Cuts) (width 0.05))
 (gr_line (start 113.792 133.096) (end 113.792 38.1) (layer Edge.Cuts) (width 0.05))
 (segment (start 160.187 116.332) (end 161.337001 117.482001) (width 0.3) (layer B.Cu) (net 1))
 (segment (start 161.60937 86.36) (end 162.687 86.36) (width 0.3) (layer B.Cu) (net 1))
 (segment (start 151.82299 89.983598) (end 155.446588 86.36) (width 0.3) (layer B.Cu) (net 1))
 (segment (start 155.446588 86.36) (end 161.60937 86.36) (width 0.3) (layer B.Cu) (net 1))
 (segment (start 159.197051 116.332) (end 151.82299 108.957939) (width 0.3) (layer B.Cu) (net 1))
 (segment (start 160.187 116.332) (end 159.197051 116.332) (width 0.3) (layer B.Cu) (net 1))
 (segment (start 192.34701 108.40001) (end 151.82299 108.40001) (width 0.3) (layer B.Cu) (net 1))
 (segment (start 195.707 111.76) (end 192.34701 108.40001) (width 0.3) (layer B.Cu) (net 1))
 (segment (start 151.82299 108.957939) (end 151.765 108.458) (width 0.3) (layer B.Cu) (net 1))
 (segment (start 151.82299 108.40001) (end 151.765 108.458) (width 0.3) (layer B.Cu) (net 1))
 (segment (start 151.765 108.458) (end 151.82299 89.983598) (width 0.3) (layer B.Cu) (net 1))
 (segment (start 133.604 74.128) (end 133.604 80.264) (width 0.3) (layer B.Cu) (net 6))
 (segment (start 134.593949 74.128) (end 134.633949 74.168) (width 0.3) (layer B.Cu) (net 6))
 (segment (start 132.804001 115.024001) (end 133.604 115.824) (width 0.3) (layer B.Cu) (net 6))
 (segment (start 132.353999 114.573999) (end 132.804001 115.024001) (width 0.3) (layer B.Cu) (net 6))
 (segment (start 132.353999 111.994001) (end 132.353999 114.573999) (width 0.3) (layer B.Cu) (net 6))
 (segment (start 133.604 110.744) (end 132.353999 111.994001) (width 0.3) (layer B.Cu) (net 6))
 (segment (start 133.604 115.824) (end 133.604 118.364) (width 0.3) (layer B.Cu) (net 6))
 (segment (start 133.604 118.364) (end 133.604 120.904) (width 0.3) (layer B.Cu) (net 6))
 (segment (start 132.353999 108.804001) (end 132.353999 81.514001) (width 0.3) (layer B.Cu) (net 6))
 (segment (start 132.353999 81.514001) (end 132.804001 81.063999) (width 0.3) (layer B.Cu) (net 6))
 (segment (start 133.604 110.054002) (end 132.353999 108.804001) (width 0.3) (layer B.Cu) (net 6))
 (segment (start 132.804001 81.063999) (end 133.604 80.264) (width 0.3) (layer B.Cu) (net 6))
 (segment (start 133.604 110.744) (end 133.604 110.054002) (width 0.3) (layer B.Cu) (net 6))
 (segment (start 183.007 111.76) (end 181.369989 110.122989) (width 0.25) (layer F.Cu) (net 36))
 (segment (start 138.062989 110.122989) (end 133.604 105.664) (width 0.25) (layer F.Cu) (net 36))
 (segment (start 181.369989 110.122989) (end 138.062989 110.122989) (width 0.25) (layer F.Cu) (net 36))
 (segment (start 185.547 111.76) (end 183.459979 109.672979) (width 0.25) (layer F.Cu) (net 34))
 (segment (start 140.152979 109.672979) (end 133.604 103.124) (width 0.25) (layer F.Cu) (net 34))
 (segment (start 183.459979 109.672979) (end 140.152979 109.672979) (width 0.25) (layer F.Cu) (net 34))
 (segment (start 188.087 111.76) (end 185.549969 109.222969) (width 0.25) (layer F.Cu) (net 32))
 (segment (start 142.242969 109.222969) (end 133.604 100.584) (width 0.25) (layer F.Cu) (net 32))
 (segment (start 185.549969 109.222969) (end 142.242969 109.222969) (width 0.25) (layer F.Cu) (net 32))
 (segment (start 190.627 111.76) (end 187.639959 108.772959) (width 0.25) (layer F.Cu) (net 30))
 (segment (start 144.332959 108.772959) (end 133.604 98.044) (width 0.25) (layer F.Cu) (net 30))
 (segment (start 187.639959 108.772959) (end 144.332959 108.772959) (width 0.25) (layer F.Cu) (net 30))
 (segment (start 176.403 113.284) (end 133.604 113.284) (width 0.25) (layer F.Cu) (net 41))
 (segment (start 177.927 111.76) (end 176.403 113.284) (width 0.25) (layer F.Cu) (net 41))
 (segment (start 178.348761 110.572999) (end 135.972999 110.572999) (width 0.25) (layer F.Cu) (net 38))
 (segment (start 180.467 111.76) (end 179.535762 111.76) (width 0.25) (layer F.Cu) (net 38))
 (segment (start 135.972999 110.572999) (end 133.604 108.204) (width 0.25) (layer F.Cu) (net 38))
 (segment (start 179.535762 111.76) (end 178.348761 110.572999) (width 0.25) (layer F.Cu) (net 38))
 (segment (start 134.403999 94.704001) (end 133.604 95.504) (width 0.25) (layer F.Cu) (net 28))
 (segment (start 140.02501 89.08299) (end 134.403999 94.704001) (width 0.25) (layer F.Cu) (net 28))
 (segment (start 192.98401 89.08299) (end 140.02501 89.08299) (width 0.25) (layer F.Cu) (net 28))
 (segment (start 195.707 86.36) (end 192.98401 89.08299) (width 0.25) (layer F.Cu) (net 28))
 (segment (start 193.167 86.36) (end 190.89402 88.63298) (width 0.25) (layer F.Cu) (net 26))
 (segment (start 137.93502 88.63298) (end 133.604 92.964) (width 0.25) (layer F.Cu) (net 26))
 (segment (start 190.89402 88.63298) (end 137.93502 88.63298) (width 0.25) (layer F.Cu) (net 26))
 (segment (start 190.627 86.36) (end 188.80403 88.18297) (width 0.25) (layer F.Cu) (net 24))
 (segment (start 135.84503 88.18297) (end 133.604 90.424) (width 0.25) (layer F.Cu) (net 24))
 (segment (start 188.80403 88.18297) (end 135.84503 88.18297) (width 0.25) (layer F.Cu) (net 24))
 (segment (start 175.387 86.36) (end 174.01404 87.73296) (width 0.25) (layer F.Cu) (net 22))
 (segment (start 134.73537 87.884) (end 133.604 87.884) (width 0.25) (layer F.Cu) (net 22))
 (segment (start 134.88641 87.73296) (end 134.73537 87.884) (width 0.25) (layer F.Cu) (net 22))
 (segment (start 174.01404 87.73296) (end 134.88641 87.73296) (width 0.25) (layer F.Cu) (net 22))
 (segment (start 133.604 123.444) (end 188.976 123.444) (width 0.25) (layer F.Cu) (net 45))
 (segment (start 193.167 119.253) (end 188.976 123.444) (width 0.25) (layer F.Cu) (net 45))
 (segment (start 193.167 111.76) (end 193.167 119.253) (width 0.25) (layer F.Cu) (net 45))
 (segment (start 198.247 111.76) (end 198.247 121.793) (width 0.25) (layer F.Cu) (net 46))
 (segment (start 194.056 125.984) (end 133.604 125.984) (width 0.25) (layer F.Cu) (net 46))
 (segment (start 198.247 121.793) (end 194.056 125.984) (width 0.25) (layer F.Cu) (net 46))
 (segment (start 162.52 111.927) (end 162.687 111.76) (width 0.3) (layer B.Cu) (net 5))
 (segment (start 162.687 115.342051) (end 162.687 111.76) (width 0.3) (layer B.Cu) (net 5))
 (segment (start 162.687 116.332) (end 162.687 115.342051) (width 0.3) (layer B.Cu) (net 5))
 (segment (start 163.703 115.316) (end 162.687 116.332) (width 0.3) (layer B.Cu) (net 5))
 (segment (start 133.604 85.344) (end 118.364 85.344) (width 0.25) (layer F.Cu) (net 3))
 (segment (start 118.364 87.884) (end 118.364 85.344) (width 0.25) (layer F.Cu) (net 3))
 (segment (start 123.968001 42.909999) (end 124.968 41.91) (width 0.25) (layer F.Cu) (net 3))
 (segment (start 117.138999 49.739001) (end 123.968001 42.909999) (width 0.25) (layer F.Cu) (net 3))
 (segment (start 117.138999 83.244001) (end 117.138999 49.739001) (width 0.25) (layer F.Cu) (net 3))
 (segment (start 118.364 84.469002) (end 117.138999 83.244001) (width 0.25) (layer F.Cu) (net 3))
 (segment (start 118.364 85.344) (end 118.364 84.469002) (width 0.25) (layer F.Cu) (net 3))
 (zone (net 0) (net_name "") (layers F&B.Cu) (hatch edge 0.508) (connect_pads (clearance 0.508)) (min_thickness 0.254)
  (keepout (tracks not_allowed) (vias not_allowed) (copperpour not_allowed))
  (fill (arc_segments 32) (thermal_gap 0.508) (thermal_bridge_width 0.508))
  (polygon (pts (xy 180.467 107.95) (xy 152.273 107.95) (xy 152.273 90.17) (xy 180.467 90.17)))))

